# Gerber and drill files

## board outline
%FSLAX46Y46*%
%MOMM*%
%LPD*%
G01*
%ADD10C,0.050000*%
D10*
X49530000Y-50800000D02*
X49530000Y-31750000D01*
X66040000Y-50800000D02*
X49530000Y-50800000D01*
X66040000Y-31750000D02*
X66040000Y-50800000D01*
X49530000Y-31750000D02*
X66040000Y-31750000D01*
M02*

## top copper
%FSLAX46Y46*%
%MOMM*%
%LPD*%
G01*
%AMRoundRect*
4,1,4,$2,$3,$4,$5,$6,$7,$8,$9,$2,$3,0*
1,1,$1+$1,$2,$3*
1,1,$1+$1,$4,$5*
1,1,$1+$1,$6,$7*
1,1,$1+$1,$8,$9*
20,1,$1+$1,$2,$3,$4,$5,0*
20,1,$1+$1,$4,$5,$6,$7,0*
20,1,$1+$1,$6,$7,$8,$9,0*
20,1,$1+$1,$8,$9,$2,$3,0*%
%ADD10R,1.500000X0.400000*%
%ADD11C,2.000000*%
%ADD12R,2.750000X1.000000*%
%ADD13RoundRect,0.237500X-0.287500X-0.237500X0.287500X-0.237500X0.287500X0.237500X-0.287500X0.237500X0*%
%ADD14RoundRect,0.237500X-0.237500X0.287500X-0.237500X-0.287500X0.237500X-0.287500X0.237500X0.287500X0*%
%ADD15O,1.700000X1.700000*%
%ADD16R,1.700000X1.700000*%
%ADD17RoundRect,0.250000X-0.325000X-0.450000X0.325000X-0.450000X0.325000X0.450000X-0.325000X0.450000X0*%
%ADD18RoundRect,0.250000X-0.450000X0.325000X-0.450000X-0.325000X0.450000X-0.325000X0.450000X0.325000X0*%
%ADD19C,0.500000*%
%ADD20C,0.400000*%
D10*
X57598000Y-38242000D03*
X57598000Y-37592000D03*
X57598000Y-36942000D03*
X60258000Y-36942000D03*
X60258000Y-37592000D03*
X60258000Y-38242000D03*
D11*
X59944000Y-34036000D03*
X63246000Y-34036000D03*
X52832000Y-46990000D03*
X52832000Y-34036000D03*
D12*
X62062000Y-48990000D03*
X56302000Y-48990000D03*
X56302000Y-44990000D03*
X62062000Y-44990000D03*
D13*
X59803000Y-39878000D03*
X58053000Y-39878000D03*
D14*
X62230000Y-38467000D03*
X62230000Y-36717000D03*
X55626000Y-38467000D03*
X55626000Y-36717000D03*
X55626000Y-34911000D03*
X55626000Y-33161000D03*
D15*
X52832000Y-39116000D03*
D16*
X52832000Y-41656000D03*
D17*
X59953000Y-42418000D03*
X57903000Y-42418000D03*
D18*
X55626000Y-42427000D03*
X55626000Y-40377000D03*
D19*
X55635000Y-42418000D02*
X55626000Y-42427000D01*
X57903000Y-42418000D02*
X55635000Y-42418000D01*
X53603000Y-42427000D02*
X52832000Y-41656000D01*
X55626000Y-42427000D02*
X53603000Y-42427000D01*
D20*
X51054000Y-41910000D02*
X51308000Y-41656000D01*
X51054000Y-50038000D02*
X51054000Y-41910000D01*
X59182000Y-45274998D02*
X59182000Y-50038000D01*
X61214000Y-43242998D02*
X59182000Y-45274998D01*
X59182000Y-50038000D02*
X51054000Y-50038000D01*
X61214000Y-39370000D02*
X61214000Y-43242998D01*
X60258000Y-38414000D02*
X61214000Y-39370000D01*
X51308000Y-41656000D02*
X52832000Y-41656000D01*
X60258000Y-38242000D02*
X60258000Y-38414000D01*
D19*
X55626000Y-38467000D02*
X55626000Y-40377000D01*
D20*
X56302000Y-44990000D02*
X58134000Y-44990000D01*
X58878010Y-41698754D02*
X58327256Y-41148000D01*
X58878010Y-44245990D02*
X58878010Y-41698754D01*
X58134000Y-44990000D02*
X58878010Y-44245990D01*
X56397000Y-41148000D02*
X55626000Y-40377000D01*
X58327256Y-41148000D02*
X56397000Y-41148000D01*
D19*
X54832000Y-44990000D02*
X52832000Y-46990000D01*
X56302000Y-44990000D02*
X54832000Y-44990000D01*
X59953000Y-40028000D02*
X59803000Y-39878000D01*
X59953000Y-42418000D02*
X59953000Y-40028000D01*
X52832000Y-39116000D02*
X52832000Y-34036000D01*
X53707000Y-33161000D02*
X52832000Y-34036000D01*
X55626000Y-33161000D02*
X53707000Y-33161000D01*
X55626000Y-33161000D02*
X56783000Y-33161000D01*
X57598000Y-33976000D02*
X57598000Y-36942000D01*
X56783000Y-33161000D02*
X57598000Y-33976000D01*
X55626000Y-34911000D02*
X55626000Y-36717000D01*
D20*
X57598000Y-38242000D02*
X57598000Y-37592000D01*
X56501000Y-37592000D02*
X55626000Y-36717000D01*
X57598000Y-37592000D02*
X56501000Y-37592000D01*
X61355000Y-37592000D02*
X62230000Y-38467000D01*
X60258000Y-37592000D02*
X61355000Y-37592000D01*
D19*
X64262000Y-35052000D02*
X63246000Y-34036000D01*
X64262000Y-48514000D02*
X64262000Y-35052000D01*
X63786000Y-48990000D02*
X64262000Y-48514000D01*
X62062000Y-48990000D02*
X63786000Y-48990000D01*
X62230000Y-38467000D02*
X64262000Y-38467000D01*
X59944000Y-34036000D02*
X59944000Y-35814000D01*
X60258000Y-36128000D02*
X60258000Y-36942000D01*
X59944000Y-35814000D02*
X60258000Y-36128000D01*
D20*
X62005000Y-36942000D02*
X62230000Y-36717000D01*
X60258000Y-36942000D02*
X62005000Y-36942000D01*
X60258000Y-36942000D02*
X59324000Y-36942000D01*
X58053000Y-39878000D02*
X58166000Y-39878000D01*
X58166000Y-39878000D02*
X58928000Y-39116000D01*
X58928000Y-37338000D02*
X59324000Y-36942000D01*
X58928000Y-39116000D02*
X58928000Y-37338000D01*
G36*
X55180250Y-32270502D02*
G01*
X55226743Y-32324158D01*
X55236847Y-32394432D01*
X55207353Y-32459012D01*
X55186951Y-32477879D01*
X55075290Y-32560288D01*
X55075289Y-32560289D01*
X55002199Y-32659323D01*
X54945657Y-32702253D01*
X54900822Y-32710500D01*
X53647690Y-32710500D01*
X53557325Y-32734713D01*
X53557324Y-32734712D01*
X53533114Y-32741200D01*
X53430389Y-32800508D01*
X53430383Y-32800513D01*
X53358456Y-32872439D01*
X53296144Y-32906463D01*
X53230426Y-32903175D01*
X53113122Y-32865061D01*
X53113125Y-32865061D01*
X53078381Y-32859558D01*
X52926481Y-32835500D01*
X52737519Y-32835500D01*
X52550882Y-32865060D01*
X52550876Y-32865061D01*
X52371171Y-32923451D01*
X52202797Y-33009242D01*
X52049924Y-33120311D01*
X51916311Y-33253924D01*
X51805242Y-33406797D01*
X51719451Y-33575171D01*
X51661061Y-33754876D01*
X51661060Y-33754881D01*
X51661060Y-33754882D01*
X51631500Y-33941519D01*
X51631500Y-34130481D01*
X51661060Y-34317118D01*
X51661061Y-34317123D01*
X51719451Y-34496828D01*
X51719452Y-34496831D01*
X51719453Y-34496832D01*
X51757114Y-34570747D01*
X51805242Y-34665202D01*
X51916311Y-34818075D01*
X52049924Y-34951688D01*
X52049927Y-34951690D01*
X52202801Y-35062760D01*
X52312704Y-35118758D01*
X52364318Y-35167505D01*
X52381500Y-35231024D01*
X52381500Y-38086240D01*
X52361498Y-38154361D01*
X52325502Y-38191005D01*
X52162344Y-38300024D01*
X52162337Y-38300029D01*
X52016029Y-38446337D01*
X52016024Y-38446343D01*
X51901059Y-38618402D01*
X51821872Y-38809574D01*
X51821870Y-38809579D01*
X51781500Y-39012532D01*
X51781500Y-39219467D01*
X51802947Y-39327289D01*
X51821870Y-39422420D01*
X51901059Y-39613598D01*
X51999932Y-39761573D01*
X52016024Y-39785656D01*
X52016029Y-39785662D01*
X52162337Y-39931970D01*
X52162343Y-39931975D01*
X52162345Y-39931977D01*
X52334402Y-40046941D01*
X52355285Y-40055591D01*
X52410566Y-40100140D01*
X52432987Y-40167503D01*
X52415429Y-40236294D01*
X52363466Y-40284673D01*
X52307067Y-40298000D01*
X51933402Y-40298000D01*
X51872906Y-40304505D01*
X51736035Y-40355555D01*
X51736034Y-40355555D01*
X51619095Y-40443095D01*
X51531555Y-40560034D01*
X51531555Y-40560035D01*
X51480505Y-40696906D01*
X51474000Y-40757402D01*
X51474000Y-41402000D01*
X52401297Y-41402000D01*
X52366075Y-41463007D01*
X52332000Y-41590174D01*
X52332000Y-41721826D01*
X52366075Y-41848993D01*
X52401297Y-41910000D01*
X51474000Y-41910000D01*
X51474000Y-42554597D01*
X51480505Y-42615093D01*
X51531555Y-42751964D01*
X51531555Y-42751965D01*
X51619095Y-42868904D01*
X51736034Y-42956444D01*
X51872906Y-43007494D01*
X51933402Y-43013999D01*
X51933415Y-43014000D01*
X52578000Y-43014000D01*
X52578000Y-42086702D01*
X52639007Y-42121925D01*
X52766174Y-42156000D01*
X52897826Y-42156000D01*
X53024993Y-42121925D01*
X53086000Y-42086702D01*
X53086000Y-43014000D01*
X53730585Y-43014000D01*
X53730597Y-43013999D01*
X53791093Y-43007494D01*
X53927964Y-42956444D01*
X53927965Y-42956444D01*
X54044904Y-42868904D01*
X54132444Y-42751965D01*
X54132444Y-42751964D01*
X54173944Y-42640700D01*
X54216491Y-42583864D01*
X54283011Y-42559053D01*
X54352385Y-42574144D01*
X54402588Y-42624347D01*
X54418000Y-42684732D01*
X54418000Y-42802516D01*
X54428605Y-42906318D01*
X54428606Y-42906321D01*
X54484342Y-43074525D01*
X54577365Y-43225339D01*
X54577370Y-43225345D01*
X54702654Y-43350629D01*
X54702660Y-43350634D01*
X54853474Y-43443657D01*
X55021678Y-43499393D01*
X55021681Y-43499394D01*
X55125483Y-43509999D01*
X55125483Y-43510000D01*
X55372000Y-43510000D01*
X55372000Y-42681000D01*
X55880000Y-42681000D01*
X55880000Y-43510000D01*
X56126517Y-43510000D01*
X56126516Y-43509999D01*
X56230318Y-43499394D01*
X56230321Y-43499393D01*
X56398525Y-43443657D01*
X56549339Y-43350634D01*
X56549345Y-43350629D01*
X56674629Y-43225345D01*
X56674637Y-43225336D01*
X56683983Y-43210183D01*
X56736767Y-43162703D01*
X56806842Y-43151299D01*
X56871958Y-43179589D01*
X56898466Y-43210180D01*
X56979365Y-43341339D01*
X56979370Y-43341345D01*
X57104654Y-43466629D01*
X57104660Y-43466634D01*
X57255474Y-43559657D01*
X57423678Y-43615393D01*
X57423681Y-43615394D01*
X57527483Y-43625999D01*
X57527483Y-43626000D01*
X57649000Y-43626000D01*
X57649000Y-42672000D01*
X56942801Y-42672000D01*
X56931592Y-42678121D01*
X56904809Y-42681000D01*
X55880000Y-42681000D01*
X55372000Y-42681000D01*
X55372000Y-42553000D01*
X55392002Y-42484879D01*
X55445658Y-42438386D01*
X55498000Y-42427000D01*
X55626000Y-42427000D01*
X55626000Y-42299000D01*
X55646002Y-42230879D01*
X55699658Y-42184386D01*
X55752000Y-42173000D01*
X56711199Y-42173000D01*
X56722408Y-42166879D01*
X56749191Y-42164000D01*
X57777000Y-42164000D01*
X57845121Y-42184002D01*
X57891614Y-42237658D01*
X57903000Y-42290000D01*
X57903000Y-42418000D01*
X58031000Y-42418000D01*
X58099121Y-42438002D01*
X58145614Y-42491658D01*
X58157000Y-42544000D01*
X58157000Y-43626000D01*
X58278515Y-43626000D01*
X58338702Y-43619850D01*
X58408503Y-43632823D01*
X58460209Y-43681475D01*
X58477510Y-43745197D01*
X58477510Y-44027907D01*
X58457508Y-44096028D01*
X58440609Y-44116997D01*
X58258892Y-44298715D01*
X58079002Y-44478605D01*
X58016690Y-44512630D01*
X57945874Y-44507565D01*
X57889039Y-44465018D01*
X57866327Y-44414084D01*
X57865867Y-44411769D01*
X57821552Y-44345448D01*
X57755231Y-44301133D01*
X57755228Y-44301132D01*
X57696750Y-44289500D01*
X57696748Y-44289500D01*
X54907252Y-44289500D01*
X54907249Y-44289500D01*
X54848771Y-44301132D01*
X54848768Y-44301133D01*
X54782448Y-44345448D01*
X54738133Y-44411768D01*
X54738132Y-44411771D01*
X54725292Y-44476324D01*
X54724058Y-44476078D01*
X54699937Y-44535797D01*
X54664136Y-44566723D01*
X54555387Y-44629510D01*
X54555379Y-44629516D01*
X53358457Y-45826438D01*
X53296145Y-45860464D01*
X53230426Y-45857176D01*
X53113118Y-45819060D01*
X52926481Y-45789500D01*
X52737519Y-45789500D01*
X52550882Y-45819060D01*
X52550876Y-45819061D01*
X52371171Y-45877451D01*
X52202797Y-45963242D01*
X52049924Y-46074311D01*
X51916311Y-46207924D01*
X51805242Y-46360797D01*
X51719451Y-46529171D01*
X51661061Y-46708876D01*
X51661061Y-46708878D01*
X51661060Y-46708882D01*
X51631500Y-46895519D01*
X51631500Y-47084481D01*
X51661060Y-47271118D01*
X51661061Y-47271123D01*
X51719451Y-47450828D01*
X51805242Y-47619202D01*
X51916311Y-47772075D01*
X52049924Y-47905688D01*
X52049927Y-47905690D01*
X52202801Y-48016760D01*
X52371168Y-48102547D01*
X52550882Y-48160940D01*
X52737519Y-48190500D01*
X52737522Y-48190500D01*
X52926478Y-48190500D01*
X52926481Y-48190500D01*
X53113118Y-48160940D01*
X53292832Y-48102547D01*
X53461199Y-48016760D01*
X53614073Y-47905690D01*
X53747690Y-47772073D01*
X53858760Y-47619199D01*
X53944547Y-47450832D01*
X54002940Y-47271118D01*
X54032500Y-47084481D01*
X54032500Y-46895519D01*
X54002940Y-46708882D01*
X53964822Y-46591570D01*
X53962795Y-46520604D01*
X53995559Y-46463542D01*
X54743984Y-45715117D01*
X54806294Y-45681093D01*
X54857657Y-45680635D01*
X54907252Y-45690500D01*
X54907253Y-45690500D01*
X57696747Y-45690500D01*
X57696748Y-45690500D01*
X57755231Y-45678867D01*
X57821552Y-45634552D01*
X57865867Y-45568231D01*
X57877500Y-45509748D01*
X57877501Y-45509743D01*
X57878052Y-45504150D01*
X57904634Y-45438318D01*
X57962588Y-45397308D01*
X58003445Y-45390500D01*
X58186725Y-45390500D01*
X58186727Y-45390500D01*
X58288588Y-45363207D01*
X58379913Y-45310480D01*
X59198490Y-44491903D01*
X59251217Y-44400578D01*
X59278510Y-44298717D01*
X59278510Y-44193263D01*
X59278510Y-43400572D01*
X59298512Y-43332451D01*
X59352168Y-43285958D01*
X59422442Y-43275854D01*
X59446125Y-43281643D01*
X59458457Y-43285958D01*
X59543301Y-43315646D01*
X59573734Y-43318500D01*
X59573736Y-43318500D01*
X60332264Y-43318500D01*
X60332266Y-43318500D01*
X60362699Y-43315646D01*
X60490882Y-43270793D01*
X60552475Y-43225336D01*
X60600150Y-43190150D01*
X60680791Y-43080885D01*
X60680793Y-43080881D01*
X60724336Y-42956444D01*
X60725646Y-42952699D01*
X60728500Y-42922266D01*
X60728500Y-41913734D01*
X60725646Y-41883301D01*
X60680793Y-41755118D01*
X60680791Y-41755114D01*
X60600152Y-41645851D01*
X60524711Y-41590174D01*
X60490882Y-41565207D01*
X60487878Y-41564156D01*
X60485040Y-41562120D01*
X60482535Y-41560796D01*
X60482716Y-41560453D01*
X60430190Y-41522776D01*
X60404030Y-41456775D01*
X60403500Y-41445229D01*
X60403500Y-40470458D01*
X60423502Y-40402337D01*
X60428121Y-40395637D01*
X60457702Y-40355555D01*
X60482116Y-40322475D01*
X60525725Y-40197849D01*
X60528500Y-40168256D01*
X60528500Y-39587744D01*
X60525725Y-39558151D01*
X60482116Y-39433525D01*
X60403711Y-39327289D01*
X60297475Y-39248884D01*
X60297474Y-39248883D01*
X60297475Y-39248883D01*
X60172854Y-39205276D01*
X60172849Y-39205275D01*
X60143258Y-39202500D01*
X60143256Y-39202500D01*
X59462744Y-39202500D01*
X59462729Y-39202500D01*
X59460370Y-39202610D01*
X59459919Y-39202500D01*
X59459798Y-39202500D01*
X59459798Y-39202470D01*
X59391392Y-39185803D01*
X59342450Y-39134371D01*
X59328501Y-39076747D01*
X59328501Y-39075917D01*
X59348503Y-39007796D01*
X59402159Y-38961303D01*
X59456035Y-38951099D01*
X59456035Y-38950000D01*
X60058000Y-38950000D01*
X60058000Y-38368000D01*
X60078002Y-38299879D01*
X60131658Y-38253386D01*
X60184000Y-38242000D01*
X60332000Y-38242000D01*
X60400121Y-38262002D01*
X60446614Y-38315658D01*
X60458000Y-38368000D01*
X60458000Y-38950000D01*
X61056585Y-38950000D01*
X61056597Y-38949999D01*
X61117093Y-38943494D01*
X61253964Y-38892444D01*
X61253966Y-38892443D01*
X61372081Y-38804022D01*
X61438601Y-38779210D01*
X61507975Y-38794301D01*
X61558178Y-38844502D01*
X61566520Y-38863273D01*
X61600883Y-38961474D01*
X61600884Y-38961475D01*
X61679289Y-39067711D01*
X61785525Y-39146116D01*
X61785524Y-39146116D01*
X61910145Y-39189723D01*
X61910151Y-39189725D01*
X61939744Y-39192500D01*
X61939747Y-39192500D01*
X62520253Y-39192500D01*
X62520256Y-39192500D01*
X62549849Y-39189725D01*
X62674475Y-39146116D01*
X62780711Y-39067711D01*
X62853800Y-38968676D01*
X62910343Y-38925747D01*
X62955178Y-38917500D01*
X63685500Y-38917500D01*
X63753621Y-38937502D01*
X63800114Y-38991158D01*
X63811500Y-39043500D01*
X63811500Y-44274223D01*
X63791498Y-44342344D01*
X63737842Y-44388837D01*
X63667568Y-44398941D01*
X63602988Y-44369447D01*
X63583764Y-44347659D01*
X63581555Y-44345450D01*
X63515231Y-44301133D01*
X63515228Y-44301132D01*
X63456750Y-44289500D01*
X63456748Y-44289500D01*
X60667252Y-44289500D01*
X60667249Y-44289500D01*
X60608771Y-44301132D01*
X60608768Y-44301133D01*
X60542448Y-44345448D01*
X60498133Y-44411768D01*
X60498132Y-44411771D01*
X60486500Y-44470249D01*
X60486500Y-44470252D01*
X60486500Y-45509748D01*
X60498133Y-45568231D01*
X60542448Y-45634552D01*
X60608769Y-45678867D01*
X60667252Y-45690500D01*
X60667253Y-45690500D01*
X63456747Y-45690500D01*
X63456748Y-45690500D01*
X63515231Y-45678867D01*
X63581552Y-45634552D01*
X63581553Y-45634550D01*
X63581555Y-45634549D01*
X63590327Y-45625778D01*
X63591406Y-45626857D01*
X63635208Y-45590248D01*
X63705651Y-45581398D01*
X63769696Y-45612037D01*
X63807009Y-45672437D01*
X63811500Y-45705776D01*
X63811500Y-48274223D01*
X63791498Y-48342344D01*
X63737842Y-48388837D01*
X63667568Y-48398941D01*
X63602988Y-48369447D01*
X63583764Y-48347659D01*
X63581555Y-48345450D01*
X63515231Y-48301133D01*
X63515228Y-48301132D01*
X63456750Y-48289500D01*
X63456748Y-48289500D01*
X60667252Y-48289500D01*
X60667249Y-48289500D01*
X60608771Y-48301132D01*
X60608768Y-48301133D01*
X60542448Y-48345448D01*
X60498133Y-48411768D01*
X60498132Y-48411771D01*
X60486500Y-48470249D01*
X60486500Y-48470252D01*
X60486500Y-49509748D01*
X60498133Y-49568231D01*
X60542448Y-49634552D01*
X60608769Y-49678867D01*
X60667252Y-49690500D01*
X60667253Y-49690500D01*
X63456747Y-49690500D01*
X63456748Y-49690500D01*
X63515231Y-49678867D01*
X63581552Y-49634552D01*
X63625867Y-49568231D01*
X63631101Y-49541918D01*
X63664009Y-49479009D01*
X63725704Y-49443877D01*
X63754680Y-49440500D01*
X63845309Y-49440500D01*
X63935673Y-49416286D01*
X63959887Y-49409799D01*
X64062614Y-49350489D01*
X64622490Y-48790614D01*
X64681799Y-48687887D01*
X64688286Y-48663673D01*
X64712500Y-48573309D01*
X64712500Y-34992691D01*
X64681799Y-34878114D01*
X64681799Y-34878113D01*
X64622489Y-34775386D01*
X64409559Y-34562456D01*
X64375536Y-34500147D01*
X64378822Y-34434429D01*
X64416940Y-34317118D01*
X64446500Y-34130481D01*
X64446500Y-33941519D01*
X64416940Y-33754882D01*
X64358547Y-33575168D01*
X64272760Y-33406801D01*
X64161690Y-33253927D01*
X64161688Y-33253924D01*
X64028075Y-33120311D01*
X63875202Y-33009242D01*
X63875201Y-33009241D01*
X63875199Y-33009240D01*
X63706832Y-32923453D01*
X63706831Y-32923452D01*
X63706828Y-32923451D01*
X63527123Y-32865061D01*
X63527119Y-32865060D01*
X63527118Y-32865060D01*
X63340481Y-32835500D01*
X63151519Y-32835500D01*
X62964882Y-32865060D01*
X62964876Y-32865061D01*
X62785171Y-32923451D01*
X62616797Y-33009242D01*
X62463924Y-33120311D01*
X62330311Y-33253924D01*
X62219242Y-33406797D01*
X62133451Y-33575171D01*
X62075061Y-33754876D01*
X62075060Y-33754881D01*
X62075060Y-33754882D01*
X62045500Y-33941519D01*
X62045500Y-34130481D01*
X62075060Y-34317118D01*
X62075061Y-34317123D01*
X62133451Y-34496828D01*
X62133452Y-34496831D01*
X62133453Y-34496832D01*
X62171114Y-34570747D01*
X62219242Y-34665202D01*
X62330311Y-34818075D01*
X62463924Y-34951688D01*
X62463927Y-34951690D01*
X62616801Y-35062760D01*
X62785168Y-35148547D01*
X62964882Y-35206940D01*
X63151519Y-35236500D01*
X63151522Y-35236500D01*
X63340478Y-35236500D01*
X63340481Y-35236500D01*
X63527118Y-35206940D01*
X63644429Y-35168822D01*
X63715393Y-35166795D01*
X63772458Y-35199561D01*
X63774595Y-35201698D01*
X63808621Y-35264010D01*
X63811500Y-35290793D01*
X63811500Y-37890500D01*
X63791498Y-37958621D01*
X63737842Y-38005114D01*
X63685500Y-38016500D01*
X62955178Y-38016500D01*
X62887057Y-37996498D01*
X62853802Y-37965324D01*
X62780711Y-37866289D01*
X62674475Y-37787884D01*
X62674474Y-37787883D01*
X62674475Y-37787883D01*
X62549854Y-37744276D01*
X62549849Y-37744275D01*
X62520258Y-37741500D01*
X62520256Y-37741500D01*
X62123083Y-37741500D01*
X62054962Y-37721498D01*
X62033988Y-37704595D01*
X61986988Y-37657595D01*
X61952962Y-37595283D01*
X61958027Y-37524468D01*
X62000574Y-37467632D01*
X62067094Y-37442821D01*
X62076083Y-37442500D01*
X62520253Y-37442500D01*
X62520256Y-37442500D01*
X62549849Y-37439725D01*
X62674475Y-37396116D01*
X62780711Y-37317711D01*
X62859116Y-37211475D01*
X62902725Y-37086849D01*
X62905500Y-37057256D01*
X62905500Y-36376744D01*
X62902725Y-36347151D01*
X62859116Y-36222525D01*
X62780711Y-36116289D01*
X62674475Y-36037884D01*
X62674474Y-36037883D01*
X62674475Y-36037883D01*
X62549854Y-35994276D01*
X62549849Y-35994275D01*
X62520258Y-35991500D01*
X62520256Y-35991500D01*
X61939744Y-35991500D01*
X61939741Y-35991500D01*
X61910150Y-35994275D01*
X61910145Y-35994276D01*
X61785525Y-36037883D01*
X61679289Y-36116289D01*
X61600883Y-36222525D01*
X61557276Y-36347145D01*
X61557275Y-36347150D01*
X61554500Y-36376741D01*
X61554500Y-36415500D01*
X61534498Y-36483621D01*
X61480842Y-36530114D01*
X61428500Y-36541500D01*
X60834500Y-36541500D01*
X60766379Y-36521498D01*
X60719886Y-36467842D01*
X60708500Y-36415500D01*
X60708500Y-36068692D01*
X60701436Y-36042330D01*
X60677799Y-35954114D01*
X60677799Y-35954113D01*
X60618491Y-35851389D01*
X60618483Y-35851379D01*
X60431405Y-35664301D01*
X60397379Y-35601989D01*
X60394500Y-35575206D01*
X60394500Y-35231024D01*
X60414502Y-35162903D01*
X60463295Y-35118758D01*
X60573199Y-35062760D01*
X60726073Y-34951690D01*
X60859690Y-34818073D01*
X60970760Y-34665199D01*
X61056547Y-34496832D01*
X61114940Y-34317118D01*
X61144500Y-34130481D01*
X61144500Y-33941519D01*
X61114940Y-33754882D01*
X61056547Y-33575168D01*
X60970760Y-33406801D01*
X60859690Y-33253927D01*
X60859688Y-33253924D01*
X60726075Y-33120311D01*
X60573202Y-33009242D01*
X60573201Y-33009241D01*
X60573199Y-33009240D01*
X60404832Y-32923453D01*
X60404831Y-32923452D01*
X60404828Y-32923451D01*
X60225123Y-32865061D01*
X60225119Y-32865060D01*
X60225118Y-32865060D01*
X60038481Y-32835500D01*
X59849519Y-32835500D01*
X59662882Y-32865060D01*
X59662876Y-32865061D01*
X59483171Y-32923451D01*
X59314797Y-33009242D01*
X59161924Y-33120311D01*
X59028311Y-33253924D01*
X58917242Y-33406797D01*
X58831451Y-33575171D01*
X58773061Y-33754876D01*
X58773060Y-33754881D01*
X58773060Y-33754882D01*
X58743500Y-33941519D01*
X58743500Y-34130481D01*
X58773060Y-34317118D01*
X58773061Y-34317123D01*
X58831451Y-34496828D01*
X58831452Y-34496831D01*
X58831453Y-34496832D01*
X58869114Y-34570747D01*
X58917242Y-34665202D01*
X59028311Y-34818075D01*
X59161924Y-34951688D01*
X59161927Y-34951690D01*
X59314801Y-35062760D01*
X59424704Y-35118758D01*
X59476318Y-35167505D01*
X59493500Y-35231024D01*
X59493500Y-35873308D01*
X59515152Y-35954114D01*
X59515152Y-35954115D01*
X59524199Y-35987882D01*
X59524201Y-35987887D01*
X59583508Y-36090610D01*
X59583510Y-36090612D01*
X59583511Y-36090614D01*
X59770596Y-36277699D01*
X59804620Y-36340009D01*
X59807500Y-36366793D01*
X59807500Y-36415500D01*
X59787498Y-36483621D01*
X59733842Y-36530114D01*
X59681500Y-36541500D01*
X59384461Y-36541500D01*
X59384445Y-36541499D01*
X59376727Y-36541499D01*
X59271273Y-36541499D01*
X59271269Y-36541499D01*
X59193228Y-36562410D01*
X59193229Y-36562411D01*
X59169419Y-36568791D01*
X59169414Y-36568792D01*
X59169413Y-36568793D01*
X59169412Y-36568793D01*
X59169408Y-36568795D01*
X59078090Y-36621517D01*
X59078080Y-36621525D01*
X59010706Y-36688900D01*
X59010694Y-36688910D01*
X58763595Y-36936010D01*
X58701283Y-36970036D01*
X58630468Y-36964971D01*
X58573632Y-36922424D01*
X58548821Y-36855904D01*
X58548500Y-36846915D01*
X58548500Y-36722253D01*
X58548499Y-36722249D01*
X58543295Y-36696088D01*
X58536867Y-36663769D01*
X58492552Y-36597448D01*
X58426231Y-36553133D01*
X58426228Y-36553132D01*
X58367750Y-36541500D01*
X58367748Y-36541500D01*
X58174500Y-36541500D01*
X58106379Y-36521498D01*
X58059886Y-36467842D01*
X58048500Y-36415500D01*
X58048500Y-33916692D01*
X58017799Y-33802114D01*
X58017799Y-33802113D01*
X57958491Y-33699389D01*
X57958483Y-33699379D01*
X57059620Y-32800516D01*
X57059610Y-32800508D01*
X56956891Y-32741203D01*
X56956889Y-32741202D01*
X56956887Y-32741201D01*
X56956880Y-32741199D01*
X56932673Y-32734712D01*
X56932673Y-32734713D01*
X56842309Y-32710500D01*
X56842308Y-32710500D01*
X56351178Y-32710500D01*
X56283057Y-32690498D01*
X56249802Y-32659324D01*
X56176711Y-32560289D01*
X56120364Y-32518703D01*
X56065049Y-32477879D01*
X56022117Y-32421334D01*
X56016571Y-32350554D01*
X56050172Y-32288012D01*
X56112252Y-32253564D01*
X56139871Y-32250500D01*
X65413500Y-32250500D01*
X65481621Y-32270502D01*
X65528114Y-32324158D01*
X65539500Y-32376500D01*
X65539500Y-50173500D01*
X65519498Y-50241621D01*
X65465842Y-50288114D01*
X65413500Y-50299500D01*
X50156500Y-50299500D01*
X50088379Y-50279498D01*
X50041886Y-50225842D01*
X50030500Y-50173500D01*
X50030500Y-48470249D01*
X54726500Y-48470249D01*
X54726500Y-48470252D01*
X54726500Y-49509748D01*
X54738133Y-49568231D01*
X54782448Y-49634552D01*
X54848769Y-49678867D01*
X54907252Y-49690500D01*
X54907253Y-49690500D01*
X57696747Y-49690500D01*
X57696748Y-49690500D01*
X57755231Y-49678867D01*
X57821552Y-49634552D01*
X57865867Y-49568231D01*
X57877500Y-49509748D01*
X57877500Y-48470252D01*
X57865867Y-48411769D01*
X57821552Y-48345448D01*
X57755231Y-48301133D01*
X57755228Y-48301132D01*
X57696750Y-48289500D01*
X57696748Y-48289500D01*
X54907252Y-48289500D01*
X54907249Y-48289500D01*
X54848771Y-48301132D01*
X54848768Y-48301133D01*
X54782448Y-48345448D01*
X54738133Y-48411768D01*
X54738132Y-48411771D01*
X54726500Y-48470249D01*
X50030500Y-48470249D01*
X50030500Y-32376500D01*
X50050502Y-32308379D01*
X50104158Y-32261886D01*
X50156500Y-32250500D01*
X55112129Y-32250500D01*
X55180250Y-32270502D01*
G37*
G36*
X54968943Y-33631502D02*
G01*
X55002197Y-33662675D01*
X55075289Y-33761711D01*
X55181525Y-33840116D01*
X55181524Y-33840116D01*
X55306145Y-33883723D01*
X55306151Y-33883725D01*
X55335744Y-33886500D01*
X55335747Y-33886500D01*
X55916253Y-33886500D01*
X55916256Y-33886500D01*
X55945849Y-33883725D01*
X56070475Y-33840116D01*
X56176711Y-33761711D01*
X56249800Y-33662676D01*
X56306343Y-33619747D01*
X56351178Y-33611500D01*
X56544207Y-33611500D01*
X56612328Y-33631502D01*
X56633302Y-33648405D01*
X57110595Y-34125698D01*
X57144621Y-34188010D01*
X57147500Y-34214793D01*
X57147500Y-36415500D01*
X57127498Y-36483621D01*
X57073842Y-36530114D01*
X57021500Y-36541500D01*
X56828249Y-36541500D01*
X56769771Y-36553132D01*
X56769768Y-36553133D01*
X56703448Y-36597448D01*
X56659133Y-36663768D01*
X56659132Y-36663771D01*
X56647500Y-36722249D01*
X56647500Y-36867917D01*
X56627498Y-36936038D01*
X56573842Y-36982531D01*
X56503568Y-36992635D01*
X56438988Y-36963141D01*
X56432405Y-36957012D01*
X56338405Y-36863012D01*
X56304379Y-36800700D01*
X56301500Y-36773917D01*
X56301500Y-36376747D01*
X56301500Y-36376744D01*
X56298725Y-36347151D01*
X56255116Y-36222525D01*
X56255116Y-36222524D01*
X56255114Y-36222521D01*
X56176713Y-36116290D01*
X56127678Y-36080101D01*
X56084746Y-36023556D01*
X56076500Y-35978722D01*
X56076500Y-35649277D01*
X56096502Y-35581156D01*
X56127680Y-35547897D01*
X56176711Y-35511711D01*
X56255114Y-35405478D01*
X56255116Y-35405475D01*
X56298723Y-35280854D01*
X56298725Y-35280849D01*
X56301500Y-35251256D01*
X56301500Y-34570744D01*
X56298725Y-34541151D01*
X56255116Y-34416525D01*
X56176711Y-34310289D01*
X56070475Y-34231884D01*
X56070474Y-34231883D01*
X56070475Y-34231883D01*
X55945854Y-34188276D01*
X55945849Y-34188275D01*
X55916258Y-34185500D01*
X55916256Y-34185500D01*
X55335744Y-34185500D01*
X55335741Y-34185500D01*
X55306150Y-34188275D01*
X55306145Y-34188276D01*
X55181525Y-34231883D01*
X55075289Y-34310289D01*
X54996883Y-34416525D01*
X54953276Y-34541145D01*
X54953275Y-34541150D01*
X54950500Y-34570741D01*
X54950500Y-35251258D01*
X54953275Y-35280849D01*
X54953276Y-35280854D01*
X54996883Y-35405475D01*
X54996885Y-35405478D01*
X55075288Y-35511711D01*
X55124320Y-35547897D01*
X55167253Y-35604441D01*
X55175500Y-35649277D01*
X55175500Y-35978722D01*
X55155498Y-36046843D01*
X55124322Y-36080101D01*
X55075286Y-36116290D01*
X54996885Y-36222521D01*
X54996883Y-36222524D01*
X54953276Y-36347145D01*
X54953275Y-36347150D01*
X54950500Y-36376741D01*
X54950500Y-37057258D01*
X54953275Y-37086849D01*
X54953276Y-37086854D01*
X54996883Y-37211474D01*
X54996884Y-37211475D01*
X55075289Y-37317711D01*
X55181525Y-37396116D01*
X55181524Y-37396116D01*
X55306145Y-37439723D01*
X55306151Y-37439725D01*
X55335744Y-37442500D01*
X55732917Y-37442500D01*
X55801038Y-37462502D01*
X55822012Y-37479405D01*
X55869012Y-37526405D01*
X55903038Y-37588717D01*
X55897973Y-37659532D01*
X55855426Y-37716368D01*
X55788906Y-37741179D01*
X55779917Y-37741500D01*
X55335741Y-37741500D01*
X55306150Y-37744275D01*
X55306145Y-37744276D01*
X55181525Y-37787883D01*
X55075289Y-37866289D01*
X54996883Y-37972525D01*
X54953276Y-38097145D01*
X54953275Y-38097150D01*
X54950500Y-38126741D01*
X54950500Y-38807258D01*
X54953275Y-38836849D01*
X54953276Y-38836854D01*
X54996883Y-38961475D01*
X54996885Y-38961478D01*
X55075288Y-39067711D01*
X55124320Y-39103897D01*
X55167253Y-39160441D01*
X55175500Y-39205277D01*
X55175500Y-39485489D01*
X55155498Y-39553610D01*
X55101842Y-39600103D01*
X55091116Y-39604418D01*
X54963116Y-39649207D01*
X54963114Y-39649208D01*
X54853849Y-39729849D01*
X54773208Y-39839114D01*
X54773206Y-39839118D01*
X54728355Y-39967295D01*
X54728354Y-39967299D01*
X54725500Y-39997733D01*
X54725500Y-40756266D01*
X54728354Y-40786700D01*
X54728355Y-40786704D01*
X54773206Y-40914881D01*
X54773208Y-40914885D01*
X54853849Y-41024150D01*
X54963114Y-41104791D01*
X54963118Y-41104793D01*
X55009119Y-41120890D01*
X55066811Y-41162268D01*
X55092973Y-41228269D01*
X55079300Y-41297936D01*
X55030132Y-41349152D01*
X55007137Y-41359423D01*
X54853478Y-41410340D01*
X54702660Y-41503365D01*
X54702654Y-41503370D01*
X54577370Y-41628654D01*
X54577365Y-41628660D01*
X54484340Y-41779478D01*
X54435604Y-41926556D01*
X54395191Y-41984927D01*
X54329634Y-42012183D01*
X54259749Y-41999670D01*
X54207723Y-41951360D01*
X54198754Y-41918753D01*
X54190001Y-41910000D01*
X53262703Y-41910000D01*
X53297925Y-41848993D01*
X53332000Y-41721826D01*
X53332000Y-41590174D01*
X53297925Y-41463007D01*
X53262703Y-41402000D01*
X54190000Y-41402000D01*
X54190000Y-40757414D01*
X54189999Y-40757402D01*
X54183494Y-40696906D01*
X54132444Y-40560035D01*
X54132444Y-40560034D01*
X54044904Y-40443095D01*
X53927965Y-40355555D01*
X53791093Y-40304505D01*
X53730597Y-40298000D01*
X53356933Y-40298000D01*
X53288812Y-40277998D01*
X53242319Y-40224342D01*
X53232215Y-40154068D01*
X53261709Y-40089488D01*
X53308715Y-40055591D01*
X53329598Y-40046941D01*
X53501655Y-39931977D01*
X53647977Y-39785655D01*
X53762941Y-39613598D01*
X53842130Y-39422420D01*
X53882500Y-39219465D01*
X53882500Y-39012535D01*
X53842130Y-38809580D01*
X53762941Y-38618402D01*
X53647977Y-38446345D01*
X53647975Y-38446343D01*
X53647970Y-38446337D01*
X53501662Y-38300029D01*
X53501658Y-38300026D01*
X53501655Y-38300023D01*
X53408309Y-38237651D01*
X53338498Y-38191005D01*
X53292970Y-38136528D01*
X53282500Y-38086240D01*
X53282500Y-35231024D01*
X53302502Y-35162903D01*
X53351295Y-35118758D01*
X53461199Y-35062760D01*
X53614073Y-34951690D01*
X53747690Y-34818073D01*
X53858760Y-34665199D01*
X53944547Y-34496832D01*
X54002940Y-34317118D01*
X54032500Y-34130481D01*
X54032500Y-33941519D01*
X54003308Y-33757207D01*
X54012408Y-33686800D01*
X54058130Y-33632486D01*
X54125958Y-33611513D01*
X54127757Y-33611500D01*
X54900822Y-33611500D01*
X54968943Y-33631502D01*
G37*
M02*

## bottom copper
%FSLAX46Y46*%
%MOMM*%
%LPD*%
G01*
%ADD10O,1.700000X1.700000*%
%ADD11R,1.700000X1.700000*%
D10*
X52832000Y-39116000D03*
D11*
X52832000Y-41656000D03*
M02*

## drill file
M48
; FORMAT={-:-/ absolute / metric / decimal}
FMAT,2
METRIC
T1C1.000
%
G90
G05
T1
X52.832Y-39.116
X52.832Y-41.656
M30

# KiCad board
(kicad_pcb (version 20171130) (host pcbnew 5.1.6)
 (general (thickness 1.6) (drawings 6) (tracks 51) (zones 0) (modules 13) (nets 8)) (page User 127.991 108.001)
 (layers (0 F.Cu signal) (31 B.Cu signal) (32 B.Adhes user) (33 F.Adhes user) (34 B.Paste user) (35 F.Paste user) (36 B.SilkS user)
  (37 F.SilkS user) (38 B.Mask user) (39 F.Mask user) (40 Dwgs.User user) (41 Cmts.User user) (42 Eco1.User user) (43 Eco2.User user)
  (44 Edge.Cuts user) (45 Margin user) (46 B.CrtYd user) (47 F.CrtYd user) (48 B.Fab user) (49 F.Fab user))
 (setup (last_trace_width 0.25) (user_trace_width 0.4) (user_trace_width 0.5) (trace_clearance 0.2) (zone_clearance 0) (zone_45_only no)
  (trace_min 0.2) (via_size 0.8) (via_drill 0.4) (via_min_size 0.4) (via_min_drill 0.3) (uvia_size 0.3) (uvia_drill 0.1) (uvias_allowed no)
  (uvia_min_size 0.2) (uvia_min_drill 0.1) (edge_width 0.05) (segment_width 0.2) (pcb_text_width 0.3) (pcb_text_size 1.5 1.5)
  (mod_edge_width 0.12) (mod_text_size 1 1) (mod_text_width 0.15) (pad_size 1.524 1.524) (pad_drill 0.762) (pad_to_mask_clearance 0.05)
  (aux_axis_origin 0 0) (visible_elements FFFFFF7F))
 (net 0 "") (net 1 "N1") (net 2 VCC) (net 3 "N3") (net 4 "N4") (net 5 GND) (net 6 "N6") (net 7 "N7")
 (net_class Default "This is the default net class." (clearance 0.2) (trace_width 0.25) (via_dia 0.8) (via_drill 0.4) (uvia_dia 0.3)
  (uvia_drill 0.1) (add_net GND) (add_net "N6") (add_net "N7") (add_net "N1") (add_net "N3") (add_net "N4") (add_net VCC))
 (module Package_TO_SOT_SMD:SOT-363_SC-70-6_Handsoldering (layer F.Cu) (at 58.928 37.592 180)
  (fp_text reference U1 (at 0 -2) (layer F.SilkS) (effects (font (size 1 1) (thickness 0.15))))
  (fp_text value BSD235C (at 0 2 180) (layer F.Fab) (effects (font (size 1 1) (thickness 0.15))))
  (pad 6 smd rect (at 1.33 -0.65 180) (size 1.5 0.4) (layers F.Cu F.Paste F.Mask) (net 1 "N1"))
  (pad 5 smd rect (at 1.33 0 180) (size 1.5 0.4) (layers F.Cu F.Paste F.Mask) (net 1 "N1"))
  (pad 4 smd rect (at 1.33 0.65 180) (size 1.5 0.4) (layers F.Cu F.Paste F.Mask) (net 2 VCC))
  (pad 3 smd rect (at -1.33 0.65 180) (size 1.5 0.4) (layers F.Cu F.Paste F.Mask) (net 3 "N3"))
  (pad 2 smd rect (at -1.33 0 180) (size 1.5 0.4) (layers F.Cu F.Paste F.Mask) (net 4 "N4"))
  (pad 1 smd rect (at -1.33 -0.65 180) (size 1.5 0.4) (layers F.Cu F.Paste F.Mask) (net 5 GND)))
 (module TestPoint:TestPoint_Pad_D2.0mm (layer F.Cu) (at 59.944 34.036)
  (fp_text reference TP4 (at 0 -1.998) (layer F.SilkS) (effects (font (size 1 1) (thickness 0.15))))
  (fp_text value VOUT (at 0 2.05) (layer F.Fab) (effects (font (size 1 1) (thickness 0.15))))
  (pad 1 smd circle (at 0 0) (size 2 2) (layers F.Cu F.Mask) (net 3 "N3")))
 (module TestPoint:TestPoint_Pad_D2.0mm (layer F.Cu) (at 63.246 34.036)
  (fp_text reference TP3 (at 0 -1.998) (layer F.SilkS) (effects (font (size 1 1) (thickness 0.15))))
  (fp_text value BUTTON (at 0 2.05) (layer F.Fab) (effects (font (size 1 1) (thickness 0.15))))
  (pad 1 smd circle (at 0 0) (size 2 2) (layers F.Cu F.Mask) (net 4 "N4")))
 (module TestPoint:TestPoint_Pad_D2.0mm (layer F.Cu) (at 52.832 46.99)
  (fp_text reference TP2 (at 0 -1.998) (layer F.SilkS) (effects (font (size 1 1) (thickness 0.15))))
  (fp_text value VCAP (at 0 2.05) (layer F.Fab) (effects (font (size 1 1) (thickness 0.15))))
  (pad 1 smd circle (at 0 0) (size 2 2) (layers F.Cu F.Mask) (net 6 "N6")))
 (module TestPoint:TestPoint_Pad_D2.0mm (layer F.Cu) (at 52.832 34.036)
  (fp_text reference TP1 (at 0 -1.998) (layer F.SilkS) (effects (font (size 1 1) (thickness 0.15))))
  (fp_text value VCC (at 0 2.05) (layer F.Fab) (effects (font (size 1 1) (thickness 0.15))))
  (pad 1 smd circle (at 0 0) (size 2 2) (layers F.Cu F.Mask) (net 2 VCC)))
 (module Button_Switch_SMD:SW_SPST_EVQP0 (layer F.Cu) (at 59.182 46.99)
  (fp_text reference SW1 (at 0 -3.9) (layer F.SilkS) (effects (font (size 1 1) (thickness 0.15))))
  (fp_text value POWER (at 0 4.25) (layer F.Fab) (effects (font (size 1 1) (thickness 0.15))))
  (pad 2 smd rect (at 2.88 2) (size 2.75 1) (layers F.Cu F.Paste F.Mask) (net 4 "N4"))
  (pad 2 smd rect (at -2.88 2) (size 2.75 1) (layers F.Cu F.Paste F.Mask) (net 4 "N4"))
  (pad 1 smd rect (at -2.88 -2) (size 2.75 1) (layers F.Cu F.Paste F.Mask) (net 6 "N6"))
  (pad 1 smd rect (at 2.88 -2) (size 2.75 1) (layers F.Cu F.Paste F.Mask) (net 6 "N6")))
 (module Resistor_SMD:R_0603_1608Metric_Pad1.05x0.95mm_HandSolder (layer F.Cu) (at 58.928 39.878)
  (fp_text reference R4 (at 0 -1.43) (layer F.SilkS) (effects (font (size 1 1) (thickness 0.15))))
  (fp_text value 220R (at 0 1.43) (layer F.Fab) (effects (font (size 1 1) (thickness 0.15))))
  (pad 2 smd roundrect (at 0.875 0) (size 1.05 0.95) (layers F.Cu F.Paste F.Mask) (roundrect_rratio 0.25) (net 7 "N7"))
  (pad 1 smd roundrect (at -0.875 0) (size 1.05 0.95) (layers F.Cu F.Paste F.Mask) (roundrect_rratio 0.25) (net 3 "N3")))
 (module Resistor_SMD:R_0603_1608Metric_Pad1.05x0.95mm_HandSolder (layer F.Cu) (at 62.23 37.592 270)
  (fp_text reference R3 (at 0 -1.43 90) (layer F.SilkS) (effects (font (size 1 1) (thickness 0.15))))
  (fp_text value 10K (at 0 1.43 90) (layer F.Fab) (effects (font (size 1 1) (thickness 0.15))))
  (pad 2 smd roundrect (at 0.875 0 270) (size 1.05 0.95) (layers F.Cu F.Paste F.Mask) (roundrect_rratio 0.25) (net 4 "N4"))
  (pad 1 smd roundrect (at -0.875 0 270) (size 1.05 0.95) (layers F.Cu F.Paste F.Mask) (roundrect_rratio 0.25) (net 3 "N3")))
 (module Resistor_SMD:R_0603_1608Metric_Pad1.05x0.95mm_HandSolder (layer F.Cu) (at 55.626 37.592 270)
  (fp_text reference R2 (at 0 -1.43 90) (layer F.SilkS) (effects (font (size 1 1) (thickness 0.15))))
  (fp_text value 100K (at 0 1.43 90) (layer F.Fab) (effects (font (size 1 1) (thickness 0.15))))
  (pad 2 smd roundrect (at 0.875 0 270) (size 1.05 0.95) (layers F.Cu F.Paste F.Mask) (roundrect_rratio 0.25) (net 6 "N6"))
  (pad 1 smd roundrect (at -0.875 0 270) (size 1.05 0.95) (layers F.Cu F.Paste F.Mask) (roundrect_rratio 0.25) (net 1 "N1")))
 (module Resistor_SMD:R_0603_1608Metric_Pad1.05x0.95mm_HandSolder (layer F.Cu) (at 55.626 34.036 270)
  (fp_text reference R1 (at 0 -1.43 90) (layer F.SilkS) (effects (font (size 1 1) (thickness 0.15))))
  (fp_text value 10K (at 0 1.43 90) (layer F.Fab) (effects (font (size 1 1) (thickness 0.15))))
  (pad 2 smd roundrect (at 0.875 0 270) (size 1.05 0.95) (layers F.Cu F.Paste F.Mask) (roundrect_rratio 0.25) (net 1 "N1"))
  (pad 1 smd roundrect (at -0.875 0 270) (size 1.05 0.95) (layers F.Cu F.Paste F.Mask) (roundrect_rratio 0.25) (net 2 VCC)))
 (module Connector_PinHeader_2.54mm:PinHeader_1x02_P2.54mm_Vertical (layer F.Cu) (at 52.832 41.656 180)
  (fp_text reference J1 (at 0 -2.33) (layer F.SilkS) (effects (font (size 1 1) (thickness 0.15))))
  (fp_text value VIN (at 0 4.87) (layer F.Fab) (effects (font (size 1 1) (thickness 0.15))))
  (pad 2 thru_hole oval (at 0 2.54 180) (size 1.7 1.7) (drill 1) (layers *.Cu *.Mask) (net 2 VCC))
  (pad 1 thru_hole rect (at 0 0 180) (size 1.7 1.7) (drill 1) (layers *.Cu *.Mask) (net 5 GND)))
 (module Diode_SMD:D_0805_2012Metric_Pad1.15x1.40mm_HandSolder (layer F.Cu) (at 58.928 42.418)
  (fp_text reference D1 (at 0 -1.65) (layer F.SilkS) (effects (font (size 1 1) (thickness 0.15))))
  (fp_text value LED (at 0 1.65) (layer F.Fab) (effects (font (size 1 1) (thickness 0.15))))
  (pad 2 smd roundrect (at 1.025 0) (size 1.15 1.4) (layers F.Cu F.Paste F.Mask) (roundrect_rratio 0.217391) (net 7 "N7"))
  (pad 1 smd roundrect (at -1.025 0) (size 1.15 1.4) (layers F.Cu F.Paste F.Mask) (roundrect_rratio 0.217391) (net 5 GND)))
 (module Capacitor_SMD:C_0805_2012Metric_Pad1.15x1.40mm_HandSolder (layer F.Cu) (at 55.626 41.402 270)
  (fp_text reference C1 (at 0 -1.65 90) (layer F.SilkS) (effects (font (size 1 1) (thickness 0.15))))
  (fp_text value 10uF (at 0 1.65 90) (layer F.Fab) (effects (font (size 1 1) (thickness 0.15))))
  (pad 2 smd roundrect (at 1.025 0 270) (size 1.15 1.4) (layers F.Cu F.Paste F.Mask) (roundrect_rratio 0.217391) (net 5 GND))
  (pad 1 smd roundrect (at -1.025 0 270) (size 1.15 1.4) (layers F.Cu F.Paste F.Mask) (roundrect_rratio 0.217391) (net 6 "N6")))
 (gr_line (start 49.53 50.8) (end 49.53 31.75) (layer Edge.Cuts) (width 0.05))
 (gr_line (start 66.04 50.8) (end 49.53 50.8) (layer Edge.Cuts) (width 0.05))
 (gr_line (start 66.04 31.75) (end 66.04 50.8) (layer Edge.Cuts) (width 0.05))
 (gr_line (start 49.53 31.75) (end 66.04 31.75) (layer Edge.Cuts) (width 0.05))
 (segment (start 55.635 42.418) (end 55.626 42.427) (width 0.5) (layer F.Cu) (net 5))
 (segment (start 57.903 42.418) (end 55.635 42.418) (width 0.5) (layer F.Cu) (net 5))
 (segment (start 53.603 42.427) (end 52.832 41.656) (width 0.5) (layer F.Cu) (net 5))
 (segment (start 55.626 42.427) (end 53.603 42.427) (width 0.5) (layer F.Cu) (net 5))
 (segment (start 51.054 41.91) (end 51.308 41.656) (width 0.4) (layer F.Cu) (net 5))
 (segment (start 51.054 50.038) (end 51.054 41.91) (width 0.4) (layer F.Cu) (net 5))
 (segment (start 59.182 45.274998) (end 59.182 50.038) (width 0.4) (layer F.Cu) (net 5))
 (segment (start 61.214 43.242998) (end 59.182 45.274998) (width 0.4) (layer F.Cu) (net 5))
 (segment (start 59.182 50.038) (end 51.054 50.038) (width 0.4) (layer F.Cu) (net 5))
 (segment (start 61.214 39.37) (end 61.214 43.242998) (width 0.4) (layer F.Cu) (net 5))
 (segment (start 60.258 38.414) (end 61.214 39.37) (width 0.4) (layer F.Cu) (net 5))
 (segment (start 51.308 41.656) (end 52.832 41.656) (width 0.4) (layer F.Cu) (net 5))
 (segment (start 60.258 38.242) (end 60.258 38.414) (width 0.4) (layer F.Cu) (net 5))
 (segment (start 55.626 38.467) (end 55.626 40.377) (width 0.5) (layer F.Cu) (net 6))
 (segment (start 56.302 44.99) (end 58.134 44.99) (width 0.4) (layer F.Cu) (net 6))
 (segment (start 58.87801 41.698754) (end 58.327256 41.148) (width 0.4) (layer F.Cu) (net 6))
 (segment (start 58.87801 44.24599) (end 58.87801 41.698754) (width 0.4) (layer F.Cu) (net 6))
 (segment (start 58.134 44.99) (end 58.87801 44.24599) (width 0.4) (layer F.Cu) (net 6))
 (segment (start 56.397 41.148) (end 55.626 40.377) (width 0.4) (layer F.Cu) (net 6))
 (segment (start 58.327256 41.148) (end 56.397 41.148) (width 0.4) (layer F.Cu) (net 6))
 (segment (start 54.832 44.99) (end 52.832 46.99) (width 0.5) (layer F.Cu) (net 6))
 (segment (start 56.302 44.99) (end 54.832 44.99) (width 0.5) (layer F.Cu) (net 6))
 (segment (start 59.953 40.028) (end 59.803 39.878) (width 0.5) (layer F.Cu) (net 7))
 (segment (start 59.953 42.418) (end 59.953 40.028) (width 0.5) (layer F.Cu) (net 7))
 (segment (start 52.832 39.116) (end 52.832 34.036) (width 0.5) (layer F.Cu) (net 2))
 (segment (start 53.707 33.161) (end 52.832 34.036) (width 0.5) (layer F.Cu) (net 2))
 (segment (start 55.626 33.161) (end 53.707 33.161) (width 0.5) (layer F.Cu) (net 2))
 (segment (start 55.626 33.161) (end 56.783 33.161) (width 0.5) (layer F.Cu) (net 2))
 (segment (start 57.598 33.976) (end 57.598 36.942) (width 0.5) (layer F.Cu) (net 2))
 (segment (start 56.783 33.161) (end 57.598 33.976) (width 0.5) (layer F.Cu) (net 2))
 (segment (start 55.626 34.911) (end 55.626 36.717) (width 0.5) (layer F.Cu) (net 1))
 (segment (start 57.598 38.242) (end 57.598 37.592) (width 0.4) (layer F.Cu) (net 1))
 (segment (start 56.501 37.592) (end 55.626 36.717) (width 0.4) (layer F.Cu) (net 1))
 (segment (start 57.598 37.592) (end 56.501 37.592) (width 0.4) (layer F.Cu) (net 1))
 (segment (start 61.355 37.592) (end 62.23 38.467) (width 0.4) (layer F.Cu) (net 4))
 (segment (start 60.258 37.592) (end 61.355 37.592) (width 0.4) (layer F.Cu) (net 4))
 (segment (start 64.262 35.052) (end 63.246 34.036) (width 0.5) (layer F.Cu) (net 4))
 (segment (start 64.262 48.514) (end 64.262 35.052) (width 0.5) (layer F.Cu) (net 4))
 (segment (start 63.786 48.99) (end 64.262 48.514) (width 0.5) (layer F.Cu) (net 4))
 (segment (start 62.062 48.99) (end 63.786 48.99) (width 0.5) (layer F.Cu) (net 4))
 (segment (start 62.23 38.467) (end 64.262 38.467) (width 0.5) (layer F.Cu) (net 4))
 (segment (start 59.944 34.036) (end 59.944 35.814) (width 0.5) (layer F.Cu) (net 3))
 (segment (start 60.258 36.128) (end 60.258 36.942) (width 0.5) (layer F.Cu) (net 3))
 (segment (start 59.944 35.814) (end 60.258 36.128) (width 0.5) (layer F.Cu) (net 3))
 (segment (start 62.005 36.942) (end 62.23 36.717) (width 0.4) (layer F.Cu) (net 3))
 (segment (start 60.258 36.942) (end 62.005 36.942) (width 0.4) (layer F.Cu) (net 3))
 (segment (start 60.258 36.942) (end 59.324 36.942) (width 0.4) (layer F.Cu) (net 3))
 (segment (start 58.053 39.878) (end 58.166 39.878) (width 0.4) (layer F.Cu) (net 3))
 (segment (start 58.166 39.878) (end 58.928 39.116) (width 0.4) (layer F.Cu) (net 3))
 (segment (start 58.928 37.338) (end 59.324 36.942) (width 0.4) (layer F.Cu) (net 3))
 (segment (start 58.928 39.116) (end 58.928 37.338) (width 0.4) (layer F.Cu) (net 3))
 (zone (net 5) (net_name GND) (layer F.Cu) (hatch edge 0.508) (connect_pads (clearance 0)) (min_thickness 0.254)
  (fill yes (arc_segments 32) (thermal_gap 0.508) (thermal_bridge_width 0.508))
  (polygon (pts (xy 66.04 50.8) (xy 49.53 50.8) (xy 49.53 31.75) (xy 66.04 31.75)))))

